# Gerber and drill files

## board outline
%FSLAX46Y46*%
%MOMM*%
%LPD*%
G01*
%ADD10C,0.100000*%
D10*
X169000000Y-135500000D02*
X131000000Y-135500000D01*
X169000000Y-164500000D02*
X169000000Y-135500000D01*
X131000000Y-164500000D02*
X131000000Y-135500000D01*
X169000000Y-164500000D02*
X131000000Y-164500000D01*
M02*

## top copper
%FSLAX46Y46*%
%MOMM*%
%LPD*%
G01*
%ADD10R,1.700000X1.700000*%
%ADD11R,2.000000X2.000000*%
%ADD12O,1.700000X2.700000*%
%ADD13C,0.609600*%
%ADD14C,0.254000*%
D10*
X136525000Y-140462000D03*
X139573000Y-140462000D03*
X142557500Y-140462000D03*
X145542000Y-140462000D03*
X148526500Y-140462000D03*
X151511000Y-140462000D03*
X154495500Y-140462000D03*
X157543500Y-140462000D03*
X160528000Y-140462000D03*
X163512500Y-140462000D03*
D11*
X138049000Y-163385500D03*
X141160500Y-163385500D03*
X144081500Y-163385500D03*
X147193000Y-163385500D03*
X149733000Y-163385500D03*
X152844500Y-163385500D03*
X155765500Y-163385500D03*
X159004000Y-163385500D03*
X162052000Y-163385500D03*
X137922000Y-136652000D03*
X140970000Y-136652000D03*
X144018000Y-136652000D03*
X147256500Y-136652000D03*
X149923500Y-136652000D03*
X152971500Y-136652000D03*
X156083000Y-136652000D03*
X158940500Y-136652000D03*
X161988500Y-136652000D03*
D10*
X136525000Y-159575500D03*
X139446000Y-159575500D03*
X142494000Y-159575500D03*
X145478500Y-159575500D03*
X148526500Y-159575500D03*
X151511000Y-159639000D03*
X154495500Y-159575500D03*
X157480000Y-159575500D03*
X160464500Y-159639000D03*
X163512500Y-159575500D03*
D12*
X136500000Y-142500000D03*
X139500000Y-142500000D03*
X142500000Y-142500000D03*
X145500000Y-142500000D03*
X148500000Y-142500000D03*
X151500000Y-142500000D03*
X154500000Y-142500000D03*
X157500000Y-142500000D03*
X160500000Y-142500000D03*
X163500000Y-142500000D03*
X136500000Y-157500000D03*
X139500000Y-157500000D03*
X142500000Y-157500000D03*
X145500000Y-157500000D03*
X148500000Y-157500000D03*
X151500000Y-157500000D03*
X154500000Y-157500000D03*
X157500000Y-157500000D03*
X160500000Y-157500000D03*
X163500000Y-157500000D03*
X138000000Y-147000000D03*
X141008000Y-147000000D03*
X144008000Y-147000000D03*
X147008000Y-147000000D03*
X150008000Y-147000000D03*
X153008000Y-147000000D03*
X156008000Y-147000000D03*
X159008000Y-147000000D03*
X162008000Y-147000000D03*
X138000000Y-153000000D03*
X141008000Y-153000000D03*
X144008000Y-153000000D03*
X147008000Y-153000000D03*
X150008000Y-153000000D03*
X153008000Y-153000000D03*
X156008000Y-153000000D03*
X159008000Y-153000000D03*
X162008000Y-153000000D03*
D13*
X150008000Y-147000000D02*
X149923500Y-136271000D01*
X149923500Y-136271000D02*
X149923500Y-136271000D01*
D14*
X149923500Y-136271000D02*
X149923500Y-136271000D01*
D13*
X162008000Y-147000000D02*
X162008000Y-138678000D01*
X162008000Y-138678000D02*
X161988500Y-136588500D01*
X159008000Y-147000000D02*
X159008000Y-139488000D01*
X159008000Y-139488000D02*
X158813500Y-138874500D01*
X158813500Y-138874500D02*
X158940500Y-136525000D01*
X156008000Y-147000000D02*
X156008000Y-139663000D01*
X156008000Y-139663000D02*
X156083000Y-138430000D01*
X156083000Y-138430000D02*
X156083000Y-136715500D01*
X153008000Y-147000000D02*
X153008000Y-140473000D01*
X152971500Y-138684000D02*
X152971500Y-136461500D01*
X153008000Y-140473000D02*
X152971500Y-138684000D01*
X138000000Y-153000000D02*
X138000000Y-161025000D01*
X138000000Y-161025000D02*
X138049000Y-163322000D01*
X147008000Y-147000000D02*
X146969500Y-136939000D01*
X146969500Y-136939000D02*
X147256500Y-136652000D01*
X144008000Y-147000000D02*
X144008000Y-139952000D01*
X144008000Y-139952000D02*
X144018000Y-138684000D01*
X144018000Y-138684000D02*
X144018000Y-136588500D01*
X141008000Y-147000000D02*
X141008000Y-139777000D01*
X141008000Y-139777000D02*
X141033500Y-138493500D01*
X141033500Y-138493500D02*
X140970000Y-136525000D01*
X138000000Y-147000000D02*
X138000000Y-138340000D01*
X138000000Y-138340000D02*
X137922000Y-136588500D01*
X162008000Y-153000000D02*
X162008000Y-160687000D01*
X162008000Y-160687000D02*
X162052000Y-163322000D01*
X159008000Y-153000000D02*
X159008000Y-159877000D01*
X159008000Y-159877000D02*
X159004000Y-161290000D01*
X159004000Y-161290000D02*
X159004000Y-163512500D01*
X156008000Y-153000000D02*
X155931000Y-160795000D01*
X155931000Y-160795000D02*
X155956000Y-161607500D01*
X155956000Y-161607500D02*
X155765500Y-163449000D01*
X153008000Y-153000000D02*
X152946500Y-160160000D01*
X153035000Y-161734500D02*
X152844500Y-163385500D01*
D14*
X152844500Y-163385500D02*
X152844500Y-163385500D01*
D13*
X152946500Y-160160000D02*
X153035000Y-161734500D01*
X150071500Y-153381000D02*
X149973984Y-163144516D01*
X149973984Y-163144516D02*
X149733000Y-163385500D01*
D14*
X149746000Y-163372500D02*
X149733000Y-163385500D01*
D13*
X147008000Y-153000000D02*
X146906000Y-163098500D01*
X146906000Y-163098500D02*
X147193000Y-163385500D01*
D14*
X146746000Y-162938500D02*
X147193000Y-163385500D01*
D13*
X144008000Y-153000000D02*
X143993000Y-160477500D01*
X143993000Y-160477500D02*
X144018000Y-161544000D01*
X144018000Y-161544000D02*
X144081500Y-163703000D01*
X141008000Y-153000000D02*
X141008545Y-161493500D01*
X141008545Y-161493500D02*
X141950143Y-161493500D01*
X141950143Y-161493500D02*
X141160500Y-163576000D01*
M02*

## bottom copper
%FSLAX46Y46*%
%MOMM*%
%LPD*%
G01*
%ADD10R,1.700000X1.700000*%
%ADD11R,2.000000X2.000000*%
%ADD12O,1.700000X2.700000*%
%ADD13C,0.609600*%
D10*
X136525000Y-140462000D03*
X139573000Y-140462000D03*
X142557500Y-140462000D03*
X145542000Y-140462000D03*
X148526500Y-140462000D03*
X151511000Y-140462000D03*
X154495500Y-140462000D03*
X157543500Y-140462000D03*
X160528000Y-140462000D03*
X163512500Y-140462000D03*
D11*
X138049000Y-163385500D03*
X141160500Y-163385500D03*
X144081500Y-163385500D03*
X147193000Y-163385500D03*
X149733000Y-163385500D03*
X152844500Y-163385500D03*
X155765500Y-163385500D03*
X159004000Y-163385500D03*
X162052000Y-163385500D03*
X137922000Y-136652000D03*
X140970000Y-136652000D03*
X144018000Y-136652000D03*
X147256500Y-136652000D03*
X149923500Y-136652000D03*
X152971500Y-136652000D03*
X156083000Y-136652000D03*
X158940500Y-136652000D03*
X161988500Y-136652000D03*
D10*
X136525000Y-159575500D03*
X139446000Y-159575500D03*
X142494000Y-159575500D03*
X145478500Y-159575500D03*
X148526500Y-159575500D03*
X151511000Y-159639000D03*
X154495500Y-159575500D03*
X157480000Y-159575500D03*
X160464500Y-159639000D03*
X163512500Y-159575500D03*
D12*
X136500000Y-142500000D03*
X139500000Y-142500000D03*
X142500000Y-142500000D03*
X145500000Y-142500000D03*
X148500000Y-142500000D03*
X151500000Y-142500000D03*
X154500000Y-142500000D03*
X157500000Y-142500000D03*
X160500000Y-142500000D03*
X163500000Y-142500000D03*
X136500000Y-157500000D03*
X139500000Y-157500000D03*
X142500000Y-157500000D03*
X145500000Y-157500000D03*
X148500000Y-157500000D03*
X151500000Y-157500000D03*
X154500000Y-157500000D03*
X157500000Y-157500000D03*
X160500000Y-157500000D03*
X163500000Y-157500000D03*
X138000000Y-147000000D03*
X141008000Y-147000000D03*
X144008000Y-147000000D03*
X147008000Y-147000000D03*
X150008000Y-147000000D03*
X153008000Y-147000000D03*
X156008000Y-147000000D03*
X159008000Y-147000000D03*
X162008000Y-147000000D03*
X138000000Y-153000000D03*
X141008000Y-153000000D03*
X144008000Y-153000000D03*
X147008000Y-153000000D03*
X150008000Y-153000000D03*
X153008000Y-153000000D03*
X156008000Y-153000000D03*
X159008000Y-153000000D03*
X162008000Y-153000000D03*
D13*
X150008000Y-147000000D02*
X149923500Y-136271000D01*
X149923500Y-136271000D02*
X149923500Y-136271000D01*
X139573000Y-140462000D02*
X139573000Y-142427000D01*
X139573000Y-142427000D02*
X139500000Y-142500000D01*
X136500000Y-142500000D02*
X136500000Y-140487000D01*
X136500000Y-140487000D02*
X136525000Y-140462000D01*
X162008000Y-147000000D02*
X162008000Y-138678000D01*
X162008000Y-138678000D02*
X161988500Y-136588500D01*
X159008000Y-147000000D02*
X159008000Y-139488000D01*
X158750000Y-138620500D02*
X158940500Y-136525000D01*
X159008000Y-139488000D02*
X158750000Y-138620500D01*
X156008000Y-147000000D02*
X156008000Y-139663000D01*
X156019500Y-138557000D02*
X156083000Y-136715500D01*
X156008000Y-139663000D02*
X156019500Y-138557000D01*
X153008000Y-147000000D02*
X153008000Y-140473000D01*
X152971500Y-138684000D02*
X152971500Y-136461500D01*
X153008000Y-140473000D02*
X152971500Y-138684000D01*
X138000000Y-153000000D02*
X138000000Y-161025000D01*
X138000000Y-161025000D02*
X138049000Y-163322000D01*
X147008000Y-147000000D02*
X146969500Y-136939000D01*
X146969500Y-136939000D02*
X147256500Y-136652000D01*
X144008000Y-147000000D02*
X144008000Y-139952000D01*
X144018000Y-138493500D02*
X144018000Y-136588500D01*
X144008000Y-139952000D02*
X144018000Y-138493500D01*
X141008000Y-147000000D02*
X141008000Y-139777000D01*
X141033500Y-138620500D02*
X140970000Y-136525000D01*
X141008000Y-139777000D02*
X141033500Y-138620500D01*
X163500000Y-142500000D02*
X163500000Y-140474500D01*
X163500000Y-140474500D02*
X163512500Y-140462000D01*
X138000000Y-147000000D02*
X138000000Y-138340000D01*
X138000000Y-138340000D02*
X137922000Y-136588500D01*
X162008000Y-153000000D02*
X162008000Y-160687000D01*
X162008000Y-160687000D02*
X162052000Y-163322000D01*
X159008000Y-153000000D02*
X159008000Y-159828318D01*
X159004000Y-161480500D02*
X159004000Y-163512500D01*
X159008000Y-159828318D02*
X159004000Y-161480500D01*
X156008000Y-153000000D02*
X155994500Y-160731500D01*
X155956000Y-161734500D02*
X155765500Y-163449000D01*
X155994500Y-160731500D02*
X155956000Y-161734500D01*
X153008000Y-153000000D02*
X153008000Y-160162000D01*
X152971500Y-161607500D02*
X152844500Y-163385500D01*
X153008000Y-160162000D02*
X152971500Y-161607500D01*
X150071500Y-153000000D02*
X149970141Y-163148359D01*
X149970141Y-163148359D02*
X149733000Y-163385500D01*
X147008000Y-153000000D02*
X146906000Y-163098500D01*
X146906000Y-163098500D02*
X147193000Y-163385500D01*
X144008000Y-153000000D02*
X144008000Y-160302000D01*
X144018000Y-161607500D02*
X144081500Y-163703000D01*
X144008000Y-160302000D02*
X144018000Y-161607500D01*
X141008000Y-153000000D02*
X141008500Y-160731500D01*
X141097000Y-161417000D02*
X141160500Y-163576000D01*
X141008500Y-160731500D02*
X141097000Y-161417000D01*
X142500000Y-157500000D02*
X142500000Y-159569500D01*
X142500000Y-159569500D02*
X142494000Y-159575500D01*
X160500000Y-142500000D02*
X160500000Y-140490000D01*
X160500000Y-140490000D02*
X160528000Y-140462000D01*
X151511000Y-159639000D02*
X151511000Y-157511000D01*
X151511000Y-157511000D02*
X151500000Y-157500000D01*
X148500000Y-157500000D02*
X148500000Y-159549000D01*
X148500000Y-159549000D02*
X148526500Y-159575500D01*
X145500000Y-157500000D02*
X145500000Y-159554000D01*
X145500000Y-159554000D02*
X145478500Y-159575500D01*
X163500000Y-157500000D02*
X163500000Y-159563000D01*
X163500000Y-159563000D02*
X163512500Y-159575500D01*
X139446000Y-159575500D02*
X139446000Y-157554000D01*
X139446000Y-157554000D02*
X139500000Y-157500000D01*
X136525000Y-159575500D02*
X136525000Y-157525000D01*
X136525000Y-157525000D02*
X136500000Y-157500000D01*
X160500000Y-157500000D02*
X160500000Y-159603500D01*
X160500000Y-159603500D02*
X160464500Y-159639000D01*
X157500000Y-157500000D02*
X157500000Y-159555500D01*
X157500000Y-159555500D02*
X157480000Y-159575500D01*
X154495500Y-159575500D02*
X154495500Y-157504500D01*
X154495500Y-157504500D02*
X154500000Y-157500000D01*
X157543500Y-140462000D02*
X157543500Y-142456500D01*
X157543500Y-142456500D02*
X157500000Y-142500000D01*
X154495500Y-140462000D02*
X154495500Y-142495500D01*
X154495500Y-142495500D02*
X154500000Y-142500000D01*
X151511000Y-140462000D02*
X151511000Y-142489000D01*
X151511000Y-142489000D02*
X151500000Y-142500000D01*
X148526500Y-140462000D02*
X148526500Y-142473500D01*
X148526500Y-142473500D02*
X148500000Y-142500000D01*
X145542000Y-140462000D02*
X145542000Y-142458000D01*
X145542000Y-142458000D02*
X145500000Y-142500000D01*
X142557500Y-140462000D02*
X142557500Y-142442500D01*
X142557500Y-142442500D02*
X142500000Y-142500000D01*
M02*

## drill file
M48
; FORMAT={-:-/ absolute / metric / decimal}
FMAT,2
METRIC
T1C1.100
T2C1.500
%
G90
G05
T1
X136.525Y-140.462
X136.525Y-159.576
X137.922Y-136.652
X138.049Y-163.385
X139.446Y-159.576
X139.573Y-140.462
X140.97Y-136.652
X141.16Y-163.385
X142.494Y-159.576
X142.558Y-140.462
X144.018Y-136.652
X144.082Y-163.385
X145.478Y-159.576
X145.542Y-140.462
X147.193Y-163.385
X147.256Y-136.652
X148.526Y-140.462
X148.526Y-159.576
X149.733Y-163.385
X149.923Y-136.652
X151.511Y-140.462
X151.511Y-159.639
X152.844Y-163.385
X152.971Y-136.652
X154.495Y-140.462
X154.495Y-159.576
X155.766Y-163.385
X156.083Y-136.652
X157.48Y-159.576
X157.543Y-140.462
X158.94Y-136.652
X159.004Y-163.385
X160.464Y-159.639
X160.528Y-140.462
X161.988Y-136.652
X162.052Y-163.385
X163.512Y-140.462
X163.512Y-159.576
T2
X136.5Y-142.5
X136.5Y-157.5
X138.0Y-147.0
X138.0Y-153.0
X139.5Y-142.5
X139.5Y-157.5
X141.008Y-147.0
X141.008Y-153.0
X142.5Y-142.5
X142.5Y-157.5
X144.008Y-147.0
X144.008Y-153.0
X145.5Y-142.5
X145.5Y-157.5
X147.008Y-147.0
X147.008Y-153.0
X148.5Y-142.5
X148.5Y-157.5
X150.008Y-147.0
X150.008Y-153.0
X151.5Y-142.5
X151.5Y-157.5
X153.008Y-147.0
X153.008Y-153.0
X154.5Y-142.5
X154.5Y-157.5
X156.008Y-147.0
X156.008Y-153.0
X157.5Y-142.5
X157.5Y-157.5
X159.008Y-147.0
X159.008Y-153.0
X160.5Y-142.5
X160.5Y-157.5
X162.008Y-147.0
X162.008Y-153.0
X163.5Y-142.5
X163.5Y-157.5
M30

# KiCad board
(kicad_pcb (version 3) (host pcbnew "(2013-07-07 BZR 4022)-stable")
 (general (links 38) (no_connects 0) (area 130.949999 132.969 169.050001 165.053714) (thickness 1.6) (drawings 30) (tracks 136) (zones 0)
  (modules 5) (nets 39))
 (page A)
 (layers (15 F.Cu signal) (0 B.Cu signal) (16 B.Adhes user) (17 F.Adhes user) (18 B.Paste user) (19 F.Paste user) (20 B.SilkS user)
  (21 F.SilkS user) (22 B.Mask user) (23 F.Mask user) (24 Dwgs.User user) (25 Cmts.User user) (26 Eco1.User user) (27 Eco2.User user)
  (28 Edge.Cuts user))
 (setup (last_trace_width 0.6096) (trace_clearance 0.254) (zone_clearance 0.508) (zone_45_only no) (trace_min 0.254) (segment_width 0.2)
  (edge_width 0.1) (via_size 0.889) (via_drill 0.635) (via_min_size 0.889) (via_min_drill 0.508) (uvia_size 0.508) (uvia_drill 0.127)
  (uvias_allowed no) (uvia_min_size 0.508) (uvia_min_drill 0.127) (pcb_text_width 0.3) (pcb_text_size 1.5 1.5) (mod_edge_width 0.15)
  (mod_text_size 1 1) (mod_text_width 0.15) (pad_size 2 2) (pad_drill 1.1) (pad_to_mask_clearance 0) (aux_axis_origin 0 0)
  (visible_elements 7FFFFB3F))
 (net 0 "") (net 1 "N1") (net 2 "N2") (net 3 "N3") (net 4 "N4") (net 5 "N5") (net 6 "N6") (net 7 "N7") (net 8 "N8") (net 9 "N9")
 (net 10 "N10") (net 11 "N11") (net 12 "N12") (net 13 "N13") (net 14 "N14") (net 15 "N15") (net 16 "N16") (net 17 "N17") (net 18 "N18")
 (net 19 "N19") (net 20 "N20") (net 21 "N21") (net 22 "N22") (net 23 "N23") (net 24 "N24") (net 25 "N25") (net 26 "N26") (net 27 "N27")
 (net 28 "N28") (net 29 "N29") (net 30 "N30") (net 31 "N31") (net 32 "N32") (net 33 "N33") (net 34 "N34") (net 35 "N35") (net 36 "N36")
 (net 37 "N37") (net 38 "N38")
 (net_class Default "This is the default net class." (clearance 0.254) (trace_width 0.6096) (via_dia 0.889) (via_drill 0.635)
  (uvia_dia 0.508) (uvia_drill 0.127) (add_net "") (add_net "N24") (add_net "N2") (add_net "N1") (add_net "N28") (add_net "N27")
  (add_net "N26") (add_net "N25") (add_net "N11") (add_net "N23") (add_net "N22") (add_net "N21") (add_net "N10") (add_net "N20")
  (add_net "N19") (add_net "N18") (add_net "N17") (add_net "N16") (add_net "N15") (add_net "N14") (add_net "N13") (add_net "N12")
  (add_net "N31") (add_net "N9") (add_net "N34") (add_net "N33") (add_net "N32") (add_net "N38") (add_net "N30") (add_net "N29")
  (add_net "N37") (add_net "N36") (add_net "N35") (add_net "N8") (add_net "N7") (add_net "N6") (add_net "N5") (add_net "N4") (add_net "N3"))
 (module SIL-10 (layer F.Cu) (at 149.733 140.462)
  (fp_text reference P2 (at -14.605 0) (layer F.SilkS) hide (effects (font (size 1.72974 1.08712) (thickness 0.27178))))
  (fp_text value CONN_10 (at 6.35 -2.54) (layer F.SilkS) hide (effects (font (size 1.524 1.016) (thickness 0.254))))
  (pad 1 thru_hole rect (at -13.208 0) (size 1.7 1.7) (drill 1.1) (layers *.Cu *.Mask F.SilkS) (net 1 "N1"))
  (pad 2 thru_hole rect (at -10.16 0) (size 1.7 1.7) (drill 1.1) (layers *.Cu *.Mask F.SilkS) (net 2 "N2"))
  (pad 3 thru_hole rect (at -7.1755 0) (size 1.7 1.7) (drill 1.1) (layers *.Cu *.Mask F.SilkS) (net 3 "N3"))
  (pad 4 thru_hole rect (at -4.191 0) (size 1.7 1.7) (drill 1.1) (layers *.Cu *.Mask F.SilkS) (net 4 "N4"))
  (pad 5 thru_hole rect (at -1.2065 0) (size 1.7 1.7) (drill 1.1) (layers *.Cu *.Mask F.SilkS) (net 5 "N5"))
  (pad 6 thru_hole rect (at 1.778 0) (size 1.7 1.7) (drill 1.1) (layers *.Cu *.Mask F.SilkS) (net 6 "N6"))
  (pad 7 thru_hole rect (at 4.7625 0) (size 1.7 1.7) (drill 1.1) (layers *.Cu *.Mask F.SilkS) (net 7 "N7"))
  (pad 8 thru_hole rect (at 7.8105 0) (size 1.7 1.7) (drill 1.1) (layers *.Cu *.Mask F.SilkS) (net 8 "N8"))
  (pad 9 thru_hole rect (at 10.795 0) (size 1.7 1.7) (drill 1.1) (layers *.Cu *.Mask F.SilkS) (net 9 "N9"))
  (pad 10 thru_hole rect (at 13.7795 0) (size 1.7 1.7) (drill 1.1) (layers *.Cu *.Mask F.SilkS) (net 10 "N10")))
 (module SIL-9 (layer F.Cu) (at 149.733 163.3855)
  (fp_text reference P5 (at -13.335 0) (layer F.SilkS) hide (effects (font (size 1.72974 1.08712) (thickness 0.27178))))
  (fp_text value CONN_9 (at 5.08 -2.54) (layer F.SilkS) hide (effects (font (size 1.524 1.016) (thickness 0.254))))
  (pad 1 thru_hole rect (at -11.684 0) (size 2 2) (drill 1.1) (layers *.Cu *.Mask F.SilkS) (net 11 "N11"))
  (pad 2 thru_hole rect (at -8.5725 0) (size 2 2) (drill 1.1) (layers *.Cu *.Mask F.SilkS) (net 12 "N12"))
  (pad 3 thru_hole rect (at -5.6515 0) (size 2 2) (drill 1.1) (layers *.Cu *.Mask F.SilkS) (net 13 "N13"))
  (pad 4 thru_hole rect (at -2.54 0) (size 2 2) (drill 1.1) (layers *.Cu *.Mask F.SilkS) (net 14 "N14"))
  (pad 5 thru_hole rect (at 0 0) (size 2 2) (drill 1.1) (layers *.Cu *.Mask F.SilkS) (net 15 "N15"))
  (pad 6 thru_hole rect (at 3.1115 0) (size 2 2) (drill 1.1) (layers *.Cu *.Mask F.SilkS) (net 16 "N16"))
  (pad 7 thru_hole rect (at 6.0325 0) (size 2 2) (drill 1.1) (layers *.Cu *.Mask F.SilkS) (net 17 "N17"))
  (pad 8 thru_hole rect (at 9.271 0) (size 2 2) (drill 1.1) (layers *.Cu *.Mask F.SilkS) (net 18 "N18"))
  (pad 9 thru_hole rect (at 12.319 0) (size 2 2) (drill 1.1) (layers *.Cu *.Mask F.SilkS) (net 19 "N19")))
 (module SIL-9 (layer F.Cu) (at 149.7965 136.652)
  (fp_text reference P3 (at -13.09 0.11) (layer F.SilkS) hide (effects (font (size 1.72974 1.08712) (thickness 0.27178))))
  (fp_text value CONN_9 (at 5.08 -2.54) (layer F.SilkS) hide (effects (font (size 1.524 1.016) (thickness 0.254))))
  (pad 1 thru_hole rect (at -11.8745 0) (size 2 2) (drill 1.1) (layers *.Cu *.Mask F.SilkS) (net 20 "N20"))
  (pad 2 thru_hole rect (at -8.8265 0) (size 2 2) (drill 1.1) (layers *.Cu *.Mask F.SilkS) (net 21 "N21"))
  (pad 3 thru_hole rect (at -5.7785 0) (size 2 2) (drill 1.1) (layers *.Cu *.Mask F.SilkS) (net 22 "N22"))
  (pad 4 thru_hole rect (at -2.54 0) (size 2 2) (drill 1.1) (layers *.Cu *.Mask F.SilkS) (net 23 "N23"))
  (pad 5 thru_hole rect (at 0.127 0) (size 2 2) (drill 1.1) (layers *.Cu *.Mask F.SilkS) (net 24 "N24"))
  (pad 6 thru_hole rect (at 3.175 0) (size 2 2) (drill 1.1) (layers *.Cu *.Mask F.SilkS) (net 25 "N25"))
  (pad 7 thru_hole rect (at 6.2865 0) (size 2 2) (drill 1.1) (layers *.Cu *.Mask F.SilkS) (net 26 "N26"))
  (pad 8 thru_hole rect (at 9.144 0) (size 2 2) (drill 1.1) (layers *.Cu *.Mask F.SilkS) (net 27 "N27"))
  (pad 9 thru_hole rect (at 12.192 0) (size 2 2) (drill 1.1) (layers *.Cu *.Mask F.SilkS) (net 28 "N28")))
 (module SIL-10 (layer F.Cu) (at 149.2885 159.5755)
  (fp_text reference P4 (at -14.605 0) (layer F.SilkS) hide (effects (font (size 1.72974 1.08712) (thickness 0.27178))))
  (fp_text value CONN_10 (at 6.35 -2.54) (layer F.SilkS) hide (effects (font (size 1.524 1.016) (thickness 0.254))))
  (pad 1 thru_hole rect (at -12.7635 0) (size 1.7 1.7) (drill 1.1) (layers *.Cu *.Mask F.SilkS) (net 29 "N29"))
  (pad 2 thru_hole rect (at -9.8425 0) (size 1.7 1.7) (drill 1.1) (layers *.Cu *.Mask F.SilkS) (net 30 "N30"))
  (pad 3 thru_hole rect (at -6.7945 0) (size 1.7 1.7) (drill 1.1) (layers *.Cu *.Mask F.SilkS) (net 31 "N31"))
  (pad 4 thru_hole rect (at -3.81 0) (size 1.7 1.7) (drill 1.1) (layers *.Cu *.Mask F.SilkS) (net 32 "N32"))
  (pad 5 thru_hole rect (at -0.762 0) (size 1.7 1.7) (drill 1.1) (layers *.Cu *.Mask F.SilkS) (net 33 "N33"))
  (pad 6 thru_hole rect (at 2.2225 0.0635) (size 1.7 1.7) (drill 1.1) (layers *.Cu *.Mask F.SilkS) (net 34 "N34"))
  (pad 7 thru_hole rect (at 5.207 0) (size 1.7 1.7) (drill 1.1) (layers *.Cu *.Mask F.SilkS) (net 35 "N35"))
  (pad 8 thru_hole rect (at 8.1915 0) (size 1.7 1.7) (drill 1.1) (layers *.Cu *.Mask F.SilkS) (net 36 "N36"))
  (pad 9 thru_hole rect (at 11.176 0.0635) (size 1.7 1.7) (drill 1.1) (layers *.Cu *.Mask F.SilkS) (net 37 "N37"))
  (pad 10 thru_hole rect (at 14.224 0) (size 1.7 1.7) (drill 1.1) (layers *.Cu *.Mask F.SilkS) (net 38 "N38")))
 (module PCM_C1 (layer F.Cu) (at 136.5 150)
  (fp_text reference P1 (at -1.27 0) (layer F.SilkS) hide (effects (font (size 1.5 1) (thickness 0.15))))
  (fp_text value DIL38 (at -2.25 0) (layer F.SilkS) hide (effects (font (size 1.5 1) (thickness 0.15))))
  (pad 1 thru_hole oval (at 0 -7.5) (size 1.7 2.7) (drill 1.5) (layers *.Cu *.Mask F.SilkS) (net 1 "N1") (zone_connect 2))
  (pad 2 thru_hole oval (at 3 -7.5) (size 1.7 2.7) (drill 1.5) (layers *.Cu *.Mask F.SilkS) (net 2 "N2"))
  (pad 3 thru_hole oval (at 6 -7.5) (size 1.7 2.7) (drill 1.5) (layers *.Cu *.Mask F.SilkS) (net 3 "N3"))
  (pad 4 thru_hole oval (at 9 -7.5) (size 1.7 2.7) (drill 1.5) (layers *.Cu *.Mask F.SilkS) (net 4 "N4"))
  (pad 5 thru_hole oval (at 12 -7.5) (size 1.7 2.7) (drill 1.5) (layers *.Cu *.Mask F.SilkS) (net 5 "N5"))
  (pad 6 thru_hole oval (at 15 -7.5) (size 1.7 2.7) (drill 1.5) (layers *.Cu *.Mask F.SilkS) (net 6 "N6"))
  (pad 7 thru_hole oval (at 18 -7.5) (size 1.7 2.7) (drill 1.5) (layers *.Cu *.Mask F.SilkS) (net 7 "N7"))
  (pad 8 thru_hole oval (at 21 -7.5) (size 1.7 2.7) (drill 1.5) (layers *.Cu *.Mask F.SilkS) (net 8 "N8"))
  (pad 9 thru_hole oval (at 24 -7.5) (size 1.7 2.7) (drill 1.5) (layers *.Cu *.Mask F.SilkS) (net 9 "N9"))
  (pad 10 thru_hole oval (at 27 -7.5) (size 1.7 2.7) (drill 1.5) (layers *.Cu *.Mask F.SilkS) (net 10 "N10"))
  (pad 29 thru_hole oval (at 0 7.5) (size 1.7 2.7) (drill 1.5) (layers *.Cu *.Mask F.SilkS) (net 29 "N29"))
  (pad 30 thru_hole oval (at 3 7.5) (size 1.7 2.7) (drill 1.5) (layers *.Cu *.Mask F.SilkS) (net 30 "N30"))
  (pad 31 thru_hole oval (at 6 7.5) (size 1.7 2.7) (drill 1.5) (layers *.Cu *.Mask F.SilkS) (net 31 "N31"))
  (pad 32 thru_hole oval (at 9 7.5) (size 1.7 2.7) (drill 1.5) (layers *.Cu *.Mask F.SilkS) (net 32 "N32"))
  (pad 33 thru_hole oval (at 12 7.5) (size 1.7 2.7) (drill 1.5) (layers *.Cu *.Mask F.SilkS) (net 33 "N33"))
  (pad 34 thru_hole oval (at 15 7.5) (size 1.7 2.7) (drill 1.5) (layers *.Cu *.Mask F.SilkS) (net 34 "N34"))
  (pad 35 thru_hole oval (at 18 7.5) (size 1.7 2.7) (drill 1.5) (layers *.Cu *.Mask F.SilkS) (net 35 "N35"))
  (pad 36 thru_hole oval (at 21 7.5) (size 1.7 2.7) (drill 1.5) (layers *.Cu *.Mask F.SilkS) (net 36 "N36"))
  (pad 37 thru_hole oval (at 24 7.5) (size 1.7 2.7) (drill 1.5) (layers *.Cu *.Mask F.SilkS) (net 37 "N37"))
  (pad 38 thru_hole oval (at 27 7.5) (size 1.7 2.7) (drill 1.5) (layers *.Cu *.Mask F.SilkS) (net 38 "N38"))
  (pad 11 thru_hole oval (at 1.5 -3) (size 1.7 2.7) (drill 1.5) (layers *.Cu *.Mask F.SilkS) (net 20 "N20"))
  (pad 12 thru_hole oval (at 4.508 -3) (size 1.7 2.7) (drill 1.5) (layers *.Cu *.Mask F.SilkS) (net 21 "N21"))
  (pad 13 thru_hole oval (at 7.508 -3) (size 1.7 2.7) (drill 1.5) (layers *.Cu *.Mask F.SilkS) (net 22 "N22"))
  (pad 14 thru_hole oval (at 10.508 -3) (size 1.7 2.7) (drill 1.5) (layers *.Cu *.Mask F.SilkS) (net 23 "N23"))
  (pad 15 thru_hole oval (at 13.508 -3) (size 1.7 2.7) (drill 1.5) (layers *.Cu *.Mask F.SilkS) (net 24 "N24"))
  (pad 16 thru_hole oval (at 16.508 -3) (size 1.7 2.7) (drill 1.5) (layers *.Cu *.Mask F.SilkS) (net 25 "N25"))
  (pad 17 thru_hole oval (at 19.508 -3) (size 1.7 2.7) (drill 1.5) (layers *.Cu *.Mask F.SilkS) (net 26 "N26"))
  (pad 18 thru_hole oval (at 22.508 -3) (size 1.7 2.7) (drill 1.5) (layers *.Cu *.Mask F.SilkS) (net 27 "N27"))
  (pad 19 thru_hole oval (at 25.508 -3) (size 1.7 2.7) (drill 1.5) (layers *.Cu *.Mask F.SilkS) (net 28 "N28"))
  (pad 20 thru_hole oval (at 1.5 3) (size 1.7 2.7) (drill 1.5) (layers *.Cu *.Mask F.SilkS) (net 11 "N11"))
  (pad 21 thru_hole oval (at 4.508 3) (size 1.7 2.7) (drill 1.5) (layers *.Cu *.Mask F.SilkS) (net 12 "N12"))
  (pad 22 thru_hole oval (at 7.508 3) (size 1.7 2.7) (drill 1.5) (layers *.Cu *.Mask F.SilkS) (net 13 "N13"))
  (pad 23 thru_hole oval (at 10.508 3) (size 1.7 2.7) (drill 1.5) (layers *.Cu *.Mask F.SilkS) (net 14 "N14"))
  (pad 24 thru_hole oval (at 13.508 3) (size 1.7 2.7) (drill 1.5) (layers *.Cu *.Mask F.SilkS) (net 15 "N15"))
  (pad 25 thru_hole oval (at 16.508 3) (size 1.7 2.7) (drill 1.5) (layers *.Cu *.Mask F.SilkS) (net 16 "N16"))
  (pad 26 thru_hole oval (at 19.508 3) (size 1.7 2.7) (drill 1.5) (layers *.Cu *.Mask F.SilkS) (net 17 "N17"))
  (pad 27 thru_hole oval (at 22.508 3) (size 1.7 2.7) (drill 1.5) (layers *.Cu *.Mask F.SilkS) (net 18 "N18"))
  (pad 28 thru_hole oval (at 25.508 3) (size 1.7 2.7) (drill 1.5) (layers *.Cu *.Mask F.SilkS) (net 19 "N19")))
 (gr_line (start 169 135.5) (end 131 135.5) (angle 90) (layer Edge.Cuts) (width 0.1))
 (gr_line (start 169 164.5) (end 169 135.5) (angle 90) (layer Edge.Cuts) (width 0.1))
 (gr_line (start 131 164.5) (end 131 135.5) (angle 90) (layer Edge.Cuts) (width 0.1))
 (gr_line (start 169 164.5) (end 131 164.5) (angle 90) (layer Edge.Cuts) (width 0.1))
 (segment (start 150.008 147) (end 149.9235 136.271) (width 0.6096) (layer F.Cu) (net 24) (status 20))
 (segment (start 149.9235 136.271) (end 149.9235 136.271) (width 0.6096) (layer F.Cu) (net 24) (status 30))
 (segment (start 150.008 147) (end 149.9235 136.271) (width 0.6096) (layer B.Cu) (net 24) (status 20))
 (segment (start 149.9235 136.271) (end 149.9235 136.271) (width 0.6096) (layer B.Cu) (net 24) (status 30))
 (segment (start 149.9235 136.271) (end 149.9235 136.271) (width 0.254) (layer F.Cu) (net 24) (status 30))
 (segment (start 139.573 140.462) (end 139.573 142.427) (width 0.6096) (layer B.Cu) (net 2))
 (segment (start 139.573 142.427) (end 139.5 142.5) (width 0.6096) (layer B.Cu) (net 2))
 (segment (start 136.5 142.5) (end 136.5 140.487) (width 0.6096) (layer B.Cu) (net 1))
 (segment (start 136.5 140.487) (end 136.525 140.462) (width 0.6096) (layer B.Cu) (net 1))
 (segment (start 162.008 147) (end 162.008 138.678) (width 0.6096) (layer F.Cu) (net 28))
 (segment (start 162.008 138.678) (end 161.9885 136.5885) (width 0.6096) (layer F.Cu) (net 28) (status 20))
 (segment (start 162.008 147) (end 162.008 138.678) (width 0.6096) (layer B.Cu) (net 28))
 (segment (start 162.008 138.678) (end 161.9885 136.5885) (width 0.6096) (layer B.Cu) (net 28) (status 20))
 (segment (start 159.008 147) (end 159.008 139.488) (width 0.6096) (layer F.Cu) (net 27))
 (segment (start 159.008 139.488) (end 158.8135 138.8745) (width 0.6096) (layer F.Cu) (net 27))
 (segment (start 158.8135 138.8745) (end 158.9405 136.525) (width 0.6096) (layer F.Cu) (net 27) (status 20))
 (segment (start 159.008 147) (end 159.008 139.488) (width 0.6096) (layer B.Cu) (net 27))
 (segment (start 158.75 138.6205) (end 158.9405 136.525) (width 0.6096) (layer B.Cu) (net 27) (status 20))
 (segment (start 159.008 139.488) (end 158.75 138.6205) (width 0.6096) (layer B.Cu) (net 27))
 (segment (start 156.008 147) (end 156.008 139.663) (width 0.6096) (layer F.Cu) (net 26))
 (segment (start 156.008 139.663) (end 156.083 138.43) (width 0.6096) (layer F.Cu) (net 26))
 (segment (start 156.083 138.43) (end 156.083 136.7155) (width 0.6096) (layer F.Cu) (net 26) (status 20))
 (segment (start 156.008 147) (end 156.008 139.663) (width 0.6096) (layer B.Cu) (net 26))
 (segment (start 156.0195 138.557) (end 156.083 136.7155) (width 0.6096) (layer B.Cu) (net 26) (status 20))
 (segment (start 156.008 139.663) (end 156.0195 138.557) (width 0.6096) (layer B.Cu) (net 26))
 (segment (start 153.008 147) (end 153.008 140.473) (width 0.6096) (layer F.Cu) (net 25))
 (segment (start 152.9715 138.684) (end 152.9715 136.4615) (width 0.6096) (layer F.Cu) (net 25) (status 20))
 (segment (start 153.008 147) (end 153.008 140.473) (width 0.6096) (layer B.Cu) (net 25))
 (segment (start 152.9715 138.684) (end 152.9715 136.4615) (width 0.6096) (layer B.Cu) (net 25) (status 20))
 (segment (start 153.008 140.473) (end 152.9715 138.684) (width 0.6096) (layer F.Cu) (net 25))
 (segment (start 153.008 140.473) (end 152.9715 138.684) (width 0.6096) (layer B.Cu) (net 25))
 (segment (start 138 153) (end 138 161.025) (width 0.6096) (layer F.Cu) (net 11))
 (segment (start 138 161.025) (end 138.049 163.322) (width 0.6096) (layer F.Cu) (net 11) (status 20))
 (segment (start 138 153) (end 138 161.025) (width 0.6096) (layer B.Cu) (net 11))
 (segment (start 138 161.025) (end 138.049 163.322) (width 0.6096) (layer B.Cu) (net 11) (status 20))
 (segment (start 147.008 147) (end 146.9695 136.939) (width 0.6096) (layer F.Cu) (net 23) (status 20))
 (segment (start 146.9695 136.939) (end 147.2565 136.652) (width 0.6096) (layer F.Cu) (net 23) (status 30))
 (segment (start 147.008 147) (end 146.9695 136.939) (width 0.6096) (layer B.Cu) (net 23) (status 20))
 (segment (start 146.9695 136.939) (end 147.2565 136.652) (width 0.6096) (layer B.Cu) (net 23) (status 30))
 (segment (start 144.008 147) (end 144.008 139.952) (width 0.6096) (layer F.Cu) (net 22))
 (segment (start 144.008 139.952) (end 144.018 138.684) (width 0.6096) (layer F.Cu) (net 22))
 (segment (start 144.018 138.684) (end 144.018 136.5885) (width 0.6096) (layer F.Cu) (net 22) (status 20))
 (segment (start 144.008 147) (end 144.008 139.952) (width 0.6096) (layer B.Cu) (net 22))
 (segment (start 144.018 138.4935) (end 144.018 136.5885) (width 0.6096) (layer B.Cu) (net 22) (status 20))
 (segment (start 144.008 139.952) (end 144.018 138.4935) (width 0.6096) (layer B.Cu) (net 22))
 (segment (start 141.008 147) (end 141.008 139.777) (width 0.6096) (layer F.Cu) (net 21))
 (segment (start 141.008 139.777) (end 141.0335 138.4935) (width 0.6096) (layer F.Cu) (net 21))
 (segment (start 141.0335 138.4935) (end 140.97 136.525) (width 0.6096) (layer F.Cu) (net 21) (status 20))
 (segment (start 141.008 147) (end 141.008 139.777) (width 0.6096) (layer B.Cu) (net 21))
 (segment (start 141.0335 138.6205) (end 140.97 136.525) (width 0.6096) (layer B.Cu) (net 21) (status 20))
 (segment (start 141.008 139.777) (end 141.0335 138.6205) (width 0.6096) (layer B.Cu) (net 21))
 (segment (start 163.5 142.5) (end 163.5 140.4745) (width 0.6096) (layer B.Cu) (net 10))
 (segment (start 163.5 140.4745) (end 163.5125 140.462) (width 0.6096) (layer B.Cu) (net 10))
 (segment (start 138 147) (end 138 138.34) (width 0.6096) (layer F.Cu) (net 20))
 (segment (start 138 138.34) (end 137.922 136.5885) (width 0.6096) (layer F.Cu) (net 20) (status 20))
 (segment (start 138 147) (end 138 138.34) (width 0.6096) (layer B.Cu) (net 20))
 (segment (start 138 138.34) (end 137.922 136.5885) (width 0.6096) (layer B.Cu) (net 20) (status 20))
 (segment (start 162.008 153) (end 162.008 160.687) (width 0.6096) (layer F.Cu) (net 19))
 (segment (start 162.008 160.687) (end 162.052 163.322) (width 0.6096) (layer F.Cu) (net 19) (status 20))
 (segment (start 162.008 153) (end 162.008 160.687) (width 0.6096) (layer B.Cu) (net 19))
 (segment (start 162.008 160.687) (end 162.052 163.322) (width 0.6096) (layer B.Cu) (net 19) (status 20))
 (segment (start 159.008 153) (end 159.008 159.877) (width 0.6096) (layer F.Cu) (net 18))
 (segment (start 159.008 159.877) (end 159.004 161.29) (width 0.6096) (layer F.Cu) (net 18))
 (segment (start 159.004 161.29) (end 159.004 163.5125) (width 0.6096) (layer F.Cu) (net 18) (status 20))
 (segment (start 159.008 153) (end 159.008 159.828318) (width 0.6096) (layer B.Cu) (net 18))
 (segment (start 159.004 161.4805) (end 159.004 163.5125) (width 0.6096) (layer B.Cu) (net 18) (status 20))
 (segment (start 159.008 159.828318) (end 159.004 161.4805) (width 0.6096) (layer B.Cu) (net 18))
 (segment (start 156.008 153) (end 155.931 160.795) (width 0.6096) (layer F.Cu) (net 17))
 (segment (start 155.931 160.795) (end 155.956 161.6075) (width 0.6096) (layer F.Cu) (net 17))
 (segment (start 155.956 161.6075) (end 155.7655 163.449) (width 0.6096) (layer F.Cu) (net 17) (status 20))
 (segment (start 156.008 153) (end 155.9945 160.7315) (width 0.6096) (layer B.Cu) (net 17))
 (segment (start 155.956 161.7345) (end 155.7655 163.449) (width 0.6096) (layer B.Cu) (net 17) (status 20))
 (segment (start 155.9945 160.7315) (end 155.956 161.7345) (width 0.6096) (layer B.Cu) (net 17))
 (segment (start 153.008 153) (end 152.9465 160.16) (width 0.6096) (layer F.Cu) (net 16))
 (segment (start 153.035 161.7345) (end 152.8445 163.3855) (width 0.6096) (layer F.Cu) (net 16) (status 20))
 (segment (start 153.008 153) (end 153.008 160.162) (width 0.6096) (layer B.Cu) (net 16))
 (segment (start 152.9715 161.6075) (end 152.8445 163.3855) (width 0.6096) (layer B.Cu) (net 16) (status 20))
 (segment (start 152.8445 163.3855) (end 152.8445 163.3855) (width 0.254) (layer F.Cu) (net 16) (status 30))
 (segment (start 152.9465 160.16) (end 153.035 161.7345) (width 0.6096) (layer F.Cu) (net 16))
 (segment (start 153.008 160.162) (end 152.9715 161.6075) (width 0.6096) (layer B.Cu) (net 16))
 (segment (start 150.0715 153.381) (end 149.973984 163.144516) (width 0.6096) (layer F.Cu) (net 15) (status 20))
 (segment (start 149.973984 163.144516) (end 149.733 163.3855) (width 0.6096) (layer F.Cu) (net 15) (status 30))
 (segment (start 150.0715 153) (end 149.970141 163.148359) (width 0.6096) (layer B.Cu) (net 15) (status 20))
 (segment (start 149.970141 163.148359) (end 149.733 163.3855) (width 0.6096) (layer B.Cu) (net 15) (status 30))
 (segment (start 149.746 163.3725) (end 149.733 163.3855) (width 0.254) (layer F.Cu) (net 15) (status 30))
 (segment (start 147.008 153) (end 146.906 163.0985) (width 0.6096) (layer F.Cu) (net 14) (status 20))
 (segment (start 146.906 163.0985) (end 147.193 163.3855) (width 0.6096) (layer F.Cu) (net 14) (status 30))
 (segment (start 147.008 153) (end 146.906 163.0985) (width 0.6096) (layer B.Cu) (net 14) (status 20))
 (segment (start 146.906 163.0985) (end 147.193 163.3855) (width 0.6096) (layer B.Cu) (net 14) (status 30))
 (segment (start 146.746 162.9385) (end 147.193 163.3855) (width 0.254) (layer F.Cu) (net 14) (status 30))
 (segment (start 144.008 153) (end 143.993 160.4775) (width 0.6096) (layer F.Cu) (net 13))
 (segment (start 143.993 160.4775) (end 144.018 161.544) (width 0.6096) (layer F.Cu) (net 13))
 (segment (start 144.018 161.544) (end 144.0815 163.703) (width 0.6096) (layer F.Cu) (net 13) (status 20))
 (segment (start 144.008 153) (end 144.008 160.302) (width 0.6096) (layer B.Cu) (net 13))
 (segment (start 144.018 161.6075) (end 144.0815 163.703) (width 0.6096) (layer B.Cu) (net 13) (status 20))
 (segment (start 144.008 160.302) (end 144.018 161.6075) (width 0.6096) (layer B.Cu) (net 13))
 (segment (start 141.008 153) (end 141.008545 161.4935) (width 0.6096) (layer F.Cu) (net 12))
 (segment (start 141.008545 161.4935) (end 141.950143 161.4935) (width 0.6096) (layer F.Cu) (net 12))
 (segment (start 141.950143 161.4935) (end 141.1605 163.576) (width 0.6096) (layer F.Cu) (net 12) (status 20))
 (segment (start 141.008 153) (end 141.0085 160.7315) (width 0.6096) (layer B.Cu) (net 12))
 (segment (start 141.097 161.417) (end 141.1605 163.576) (width 0.6096) (layer B.Cu) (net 12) (status 20))
 (segment (start 141.0085 160.7315) (end 141.097 161.417) (width 0.6096) (layer B.Cu) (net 12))
 (segment (start 142.5 157.5) (end 142.5 159.5695) (width 0.6096) (layer B.Cu) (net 31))
 (segment (start 142.5 159.5695) (end 142.494 159.5755) (width 0.6096) (layer B.Cu) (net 31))
 (segment (start 160.5 142.5) (end 160.5 140.49) (width 0.6096) (layer B.Cu) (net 9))
 (segment (start 160.5 140.49) (end 160.528 140.462) (width 0.6096) (layer B.Cu) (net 9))
 (segment (start 151.511 159.639) (end 151.511 157.511) (width 0.6096) (layer B.Cu) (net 34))
 (segment (start 151.511 157.511) (end 151.5 157.5) (width 0.6096) (layer B.Cu) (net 34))
 (segment (start 148.5 157.5) (end 148.5 159.549) (width 0.6096) (layer B.Cu) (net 33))
 (segment (start 148.5 159.549) (end 148.5265 159.5755) (width 0.6096) (layer B.Cu) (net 33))
 (segment (start 145.5 157.5) (end 145.5 159.554) (width 0.6096) (layer B.Cu) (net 32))
 (segment (start 145.5 159.554) (end 145.4785 159.5755) (width 0.6096) (layer B.Cu) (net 32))
 (segment (start 163.5 157.5) (end 163.5 159.563) (width 0.6096) (layer B.Cu) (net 38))
 (segment (start 163.5 159.563) (end 163.5125 159.5755) (width 0.6096) (layer B.Cu) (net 38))
 (segment (start 139.446 159.5755) (end 139.446 157.554) (width 0.6096) (layer B.Cu) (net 30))
 (segment (start 139.446 157.554) (end 139.5 157.5) (width 0.6096) (layer B.Cu) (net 30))
 (segment (start 136.525 159.5755) (end 136.525 157.525) (width 0.6096) (layer B.Cu) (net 29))
 (segment (start 136.525 157.525) (end 136.5 157.5) (width 0.6096) (layer B.Cu) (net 29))
 (segment (start 160.5 157.5) (end 160.5 159.6035) (width 0.6096) (layer B.Cu) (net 37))
 (segment (start 160.5 159.6035) (end 160.4645 159.639) (width 0.6096) (layer B.Cu) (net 37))
 (segment (start 157.5 157.5) (end 157.5 159.5555) (width 0.6096) (layer B.Cu) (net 36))
 (segment (start 157.5 159.5555) (end 157.48 159.5755) (width 0.6096) (layer B.Cu) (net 36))
 (segment (start 154.4955 159.5755) (end 154.4955 157.5045) (width 0.6096) (layer B.Cu) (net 35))
 (segment (start 154.4955 157.5045) (end 154.5 157.5) (width 0.6096) (layer B.Cu) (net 35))
 (segment (start 157.5435 140.462) (end 157.5435 142.4565) (width 0.6096) (layer B.Cu) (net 8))
 (segment (start 157.5435 142.4565) (end 157.5 142.5) (width 0.6096) (layer B.Cu) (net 8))
 (segment (start 154.4955 140.462) (end 154.4955 142.4955) (width 0.6096) (layer B.Cu) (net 7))
 (segment (start 154.4955 142.4955) (end 154.5 142.5) (width 0.6096) (layer B.Cu) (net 7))
 (segment (start 151.511 140.462) (end 151.511 142.489) (width 0.6096) (layer B.Cu) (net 6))
 (segment (start 151.511 142.489) (end 151.5 142.5) (width 0.6096) (layer B.Cu) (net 6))
 (segment (start 148.5265 140.462) (end 148.5265 142.4735) (width 0.6096) (layer B.Cu) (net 5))
 (segment (start 148.5265 142.4735) (end 148.5 142.5) (width 0.6096) (layer B.Cu) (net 5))
 (segment (start 145.542 140.462) (end 145.542 142.458) (width 0.6096) (layer B.Cu) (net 4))
 (segment (start 145.542 142.458) (end 145.5 142.5) (width 0.6096) (layer B.Cu) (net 4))
 (segment (start 142.5575 140.462) (end 142.5575 142.4425) (width 0.6096) (layer B.Cu) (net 3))
 (segment (start 142.5575 142.4425) (end 142.5 142.5) (width 0.6096) (layer B.Cu) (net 3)))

